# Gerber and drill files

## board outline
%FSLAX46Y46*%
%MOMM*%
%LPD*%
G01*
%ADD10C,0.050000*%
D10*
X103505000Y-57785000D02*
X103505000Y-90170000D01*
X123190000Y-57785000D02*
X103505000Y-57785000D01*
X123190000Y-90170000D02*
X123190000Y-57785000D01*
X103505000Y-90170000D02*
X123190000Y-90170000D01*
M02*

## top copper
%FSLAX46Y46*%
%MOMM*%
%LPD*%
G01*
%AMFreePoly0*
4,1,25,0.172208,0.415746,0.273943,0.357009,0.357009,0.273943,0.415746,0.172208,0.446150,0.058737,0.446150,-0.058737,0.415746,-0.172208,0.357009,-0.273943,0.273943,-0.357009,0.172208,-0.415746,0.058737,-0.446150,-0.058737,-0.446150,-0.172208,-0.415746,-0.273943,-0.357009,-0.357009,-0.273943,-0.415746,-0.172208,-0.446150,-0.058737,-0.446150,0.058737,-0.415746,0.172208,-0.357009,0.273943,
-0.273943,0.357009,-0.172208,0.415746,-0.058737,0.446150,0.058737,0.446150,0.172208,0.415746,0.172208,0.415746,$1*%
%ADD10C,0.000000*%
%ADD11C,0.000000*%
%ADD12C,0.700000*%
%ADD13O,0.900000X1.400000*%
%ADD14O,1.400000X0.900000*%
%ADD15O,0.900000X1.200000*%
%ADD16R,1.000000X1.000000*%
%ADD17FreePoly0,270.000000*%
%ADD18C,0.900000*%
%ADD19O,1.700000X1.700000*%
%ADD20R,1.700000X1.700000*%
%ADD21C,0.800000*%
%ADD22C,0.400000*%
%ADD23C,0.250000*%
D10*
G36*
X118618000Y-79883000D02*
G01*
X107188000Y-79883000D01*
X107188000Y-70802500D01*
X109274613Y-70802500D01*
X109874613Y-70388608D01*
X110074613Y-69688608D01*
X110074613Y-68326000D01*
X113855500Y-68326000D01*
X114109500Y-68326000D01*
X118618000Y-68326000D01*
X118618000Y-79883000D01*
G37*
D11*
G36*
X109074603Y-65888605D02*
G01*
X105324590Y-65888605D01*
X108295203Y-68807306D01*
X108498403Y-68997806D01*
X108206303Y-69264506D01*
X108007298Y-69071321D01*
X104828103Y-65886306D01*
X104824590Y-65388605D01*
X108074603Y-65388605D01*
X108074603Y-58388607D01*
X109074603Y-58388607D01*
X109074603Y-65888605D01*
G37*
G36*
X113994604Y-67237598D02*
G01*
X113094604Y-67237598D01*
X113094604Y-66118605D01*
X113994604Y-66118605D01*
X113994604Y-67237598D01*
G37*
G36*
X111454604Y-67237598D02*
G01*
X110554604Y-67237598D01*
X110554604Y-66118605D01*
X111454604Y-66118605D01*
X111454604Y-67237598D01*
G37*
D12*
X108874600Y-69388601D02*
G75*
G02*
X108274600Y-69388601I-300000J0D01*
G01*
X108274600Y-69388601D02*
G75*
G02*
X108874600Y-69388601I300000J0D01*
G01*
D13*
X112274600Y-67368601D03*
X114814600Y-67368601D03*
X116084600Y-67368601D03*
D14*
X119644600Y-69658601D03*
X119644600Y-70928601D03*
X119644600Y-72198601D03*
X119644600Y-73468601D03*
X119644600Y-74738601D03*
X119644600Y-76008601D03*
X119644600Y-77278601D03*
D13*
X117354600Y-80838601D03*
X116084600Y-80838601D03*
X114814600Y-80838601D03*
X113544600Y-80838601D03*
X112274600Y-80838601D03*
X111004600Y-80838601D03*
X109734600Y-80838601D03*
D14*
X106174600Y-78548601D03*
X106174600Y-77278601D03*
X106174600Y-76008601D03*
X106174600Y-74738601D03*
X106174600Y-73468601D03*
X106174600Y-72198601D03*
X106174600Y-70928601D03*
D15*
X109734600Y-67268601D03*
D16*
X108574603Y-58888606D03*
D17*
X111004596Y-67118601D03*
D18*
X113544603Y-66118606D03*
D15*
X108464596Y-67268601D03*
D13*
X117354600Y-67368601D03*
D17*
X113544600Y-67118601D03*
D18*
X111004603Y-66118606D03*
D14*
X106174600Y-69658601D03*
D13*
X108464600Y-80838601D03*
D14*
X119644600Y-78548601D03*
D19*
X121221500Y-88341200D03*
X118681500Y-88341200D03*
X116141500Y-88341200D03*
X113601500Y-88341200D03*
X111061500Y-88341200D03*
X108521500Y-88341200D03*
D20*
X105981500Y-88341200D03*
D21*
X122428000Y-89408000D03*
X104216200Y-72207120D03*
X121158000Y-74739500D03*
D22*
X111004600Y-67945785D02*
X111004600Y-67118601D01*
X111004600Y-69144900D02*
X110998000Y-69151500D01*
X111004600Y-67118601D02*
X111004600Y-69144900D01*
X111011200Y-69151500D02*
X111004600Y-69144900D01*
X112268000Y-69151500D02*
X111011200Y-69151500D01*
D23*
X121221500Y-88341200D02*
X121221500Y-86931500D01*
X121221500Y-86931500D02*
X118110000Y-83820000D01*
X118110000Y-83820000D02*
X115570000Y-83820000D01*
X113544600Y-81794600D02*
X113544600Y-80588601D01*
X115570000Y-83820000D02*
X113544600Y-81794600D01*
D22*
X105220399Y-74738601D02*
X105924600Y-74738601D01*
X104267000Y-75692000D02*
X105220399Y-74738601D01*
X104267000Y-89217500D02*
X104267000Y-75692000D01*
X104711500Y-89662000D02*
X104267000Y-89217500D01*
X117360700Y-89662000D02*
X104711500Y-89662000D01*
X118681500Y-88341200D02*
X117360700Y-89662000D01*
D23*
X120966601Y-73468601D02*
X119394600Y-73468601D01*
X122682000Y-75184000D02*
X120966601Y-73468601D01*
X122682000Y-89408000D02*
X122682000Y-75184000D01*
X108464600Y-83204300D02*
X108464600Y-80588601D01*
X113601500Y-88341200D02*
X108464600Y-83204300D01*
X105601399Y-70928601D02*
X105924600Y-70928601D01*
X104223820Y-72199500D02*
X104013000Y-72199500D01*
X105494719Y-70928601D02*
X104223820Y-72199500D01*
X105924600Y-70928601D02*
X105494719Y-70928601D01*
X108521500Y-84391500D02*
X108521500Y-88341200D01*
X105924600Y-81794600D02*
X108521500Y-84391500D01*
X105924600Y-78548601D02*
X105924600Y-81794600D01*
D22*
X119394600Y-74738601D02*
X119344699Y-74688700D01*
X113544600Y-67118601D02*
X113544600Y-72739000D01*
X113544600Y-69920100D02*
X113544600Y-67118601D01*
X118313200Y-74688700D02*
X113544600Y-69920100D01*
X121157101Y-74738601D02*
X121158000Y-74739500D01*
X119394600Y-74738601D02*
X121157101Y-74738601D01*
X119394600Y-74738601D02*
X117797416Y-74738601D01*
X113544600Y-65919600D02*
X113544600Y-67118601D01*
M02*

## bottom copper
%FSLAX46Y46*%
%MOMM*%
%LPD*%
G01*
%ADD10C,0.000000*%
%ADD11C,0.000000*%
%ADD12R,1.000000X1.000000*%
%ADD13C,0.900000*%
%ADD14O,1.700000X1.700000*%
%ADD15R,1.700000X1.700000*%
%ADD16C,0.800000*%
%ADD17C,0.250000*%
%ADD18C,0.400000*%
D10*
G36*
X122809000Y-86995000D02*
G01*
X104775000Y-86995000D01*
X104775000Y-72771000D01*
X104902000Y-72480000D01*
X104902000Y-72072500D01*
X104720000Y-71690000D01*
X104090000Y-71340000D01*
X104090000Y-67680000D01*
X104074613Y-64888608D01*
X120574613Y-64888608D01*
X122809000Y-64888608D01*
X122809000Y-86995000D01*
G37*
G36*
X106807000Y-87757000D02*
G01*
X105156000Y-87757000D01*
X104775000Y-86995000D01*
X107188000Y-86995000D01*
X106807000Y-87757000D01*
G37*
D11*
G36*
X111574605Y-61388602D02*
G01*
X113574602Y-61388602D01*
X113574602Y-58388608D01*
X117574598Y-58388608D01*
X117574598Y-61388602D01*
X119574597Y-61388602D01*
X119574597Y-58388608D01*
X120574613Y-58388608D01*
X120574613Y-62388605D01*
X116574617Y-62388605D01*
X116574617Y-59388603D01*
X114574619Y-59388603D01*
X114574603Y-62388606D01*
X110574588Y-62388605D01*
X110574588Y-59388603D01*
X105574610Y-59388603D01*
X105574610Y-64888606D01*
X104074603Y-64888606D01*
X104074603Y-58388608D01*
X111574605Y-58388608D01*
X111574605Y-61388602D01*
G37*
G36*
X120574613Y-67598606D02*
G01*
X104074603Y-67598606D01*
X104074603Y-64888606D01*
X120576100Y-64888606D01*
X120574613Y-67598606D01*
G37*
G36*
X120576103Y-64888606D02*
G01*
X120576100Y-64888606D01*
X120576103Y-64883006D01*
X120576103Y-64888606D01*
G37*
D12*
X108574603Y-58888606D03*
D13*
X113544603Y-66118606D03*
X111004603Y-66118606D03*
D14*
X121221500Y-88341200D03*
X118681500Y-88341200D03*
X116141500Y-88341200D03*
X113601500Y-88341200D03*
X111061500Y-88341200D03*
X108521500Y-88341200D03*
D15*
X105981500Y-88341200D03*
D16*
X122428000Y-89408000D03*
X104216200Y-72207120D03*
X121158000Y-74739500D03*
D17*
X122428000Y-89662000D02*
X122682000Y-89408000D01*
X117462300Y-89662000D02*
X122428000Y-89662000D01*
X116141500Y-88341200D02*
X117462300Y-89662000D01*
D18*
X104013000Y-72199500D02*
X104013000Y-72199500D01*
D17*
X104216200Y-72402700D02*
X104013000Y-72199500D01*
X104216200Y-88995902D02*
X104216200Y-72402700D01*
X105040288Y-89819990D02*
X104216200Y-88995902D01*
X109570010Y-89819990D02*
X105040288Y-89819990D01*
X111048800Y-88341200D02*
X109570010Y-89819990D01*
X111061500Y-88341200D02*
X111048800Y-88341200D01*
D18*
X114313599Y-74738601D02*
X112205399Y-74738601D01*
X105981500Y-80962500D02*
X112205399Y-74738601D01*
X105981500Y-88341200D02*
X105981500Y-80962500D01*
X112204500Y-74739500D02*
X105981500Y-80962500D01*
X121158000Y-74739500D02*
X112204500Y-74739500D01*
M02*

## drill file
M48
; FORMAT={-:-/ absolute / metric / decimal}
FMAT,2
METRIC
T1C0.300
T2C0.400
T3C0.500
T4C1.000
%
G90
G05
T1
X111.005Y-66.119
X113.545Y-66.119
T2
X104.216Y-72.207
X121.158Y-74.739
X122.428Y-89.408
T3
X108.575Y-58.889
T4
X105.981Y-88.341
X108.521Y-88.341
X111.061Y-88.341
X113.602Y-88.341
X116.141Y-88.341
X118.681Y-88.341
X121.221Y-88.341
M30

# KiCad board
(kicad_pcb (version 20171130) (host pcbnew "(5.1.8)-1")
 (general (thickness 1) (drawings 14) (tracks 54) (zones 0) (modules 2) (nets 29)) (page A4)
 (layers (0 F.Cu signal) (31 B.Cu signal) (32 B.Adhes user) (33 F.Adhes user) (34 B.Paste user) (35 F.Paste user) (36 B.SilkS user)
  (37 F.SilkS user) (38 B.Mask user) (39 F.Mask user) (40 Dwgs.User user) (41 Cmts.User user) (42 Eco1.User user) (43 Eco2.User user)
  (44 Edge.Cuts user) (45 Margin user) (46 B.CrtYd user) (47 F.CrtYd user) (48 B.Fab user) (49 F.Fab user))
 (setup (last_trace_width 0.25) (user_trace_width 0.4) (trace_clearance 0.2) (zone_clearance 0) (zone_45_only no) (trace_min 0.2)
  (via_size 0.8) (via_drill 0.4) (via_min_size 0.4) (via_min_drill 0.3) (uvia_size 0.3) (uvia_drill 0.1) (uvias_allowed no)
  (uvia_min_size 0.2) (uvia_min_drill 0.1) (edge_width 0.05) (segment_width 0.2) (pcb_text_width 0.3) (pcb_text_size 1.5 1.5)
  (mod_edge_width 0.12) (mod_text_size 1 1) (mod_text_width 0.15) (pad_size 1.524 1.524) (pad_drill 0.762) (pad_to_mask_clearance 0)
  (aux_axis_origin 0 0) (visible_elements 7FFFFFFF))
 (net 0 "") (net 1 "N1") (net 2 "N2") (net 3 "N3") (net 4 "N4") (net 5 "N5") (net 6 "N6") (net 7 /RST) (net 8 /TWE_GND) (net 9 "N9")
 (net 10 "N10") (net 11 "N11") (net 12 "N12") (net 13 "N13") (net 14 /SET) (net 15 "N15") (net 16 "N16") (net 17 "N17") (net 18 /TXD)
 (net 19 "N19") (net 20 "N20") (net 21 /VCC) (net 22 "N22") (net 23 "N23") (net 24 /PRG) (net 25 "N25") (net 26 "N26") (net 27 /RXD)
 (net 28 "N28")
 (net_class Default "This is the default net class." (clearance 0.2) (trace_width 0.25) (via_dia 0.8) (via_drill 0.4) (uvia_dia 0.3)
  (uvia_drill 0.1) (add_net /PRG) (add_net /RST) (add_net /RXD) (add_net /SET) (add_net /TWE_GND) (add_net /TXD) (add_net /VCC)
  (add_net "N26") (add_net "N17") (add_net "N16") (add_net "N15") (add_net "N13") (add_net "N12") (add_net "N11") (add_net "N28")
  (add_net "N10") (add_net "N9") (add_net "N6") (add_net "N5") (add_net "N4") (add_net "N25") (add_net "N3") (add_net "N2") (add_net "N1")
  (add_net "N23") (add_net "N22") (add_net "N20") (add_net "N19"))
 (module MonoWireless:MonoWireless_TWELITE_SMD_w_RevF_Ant (layer F.Cu) (at 112.9096 74.103601)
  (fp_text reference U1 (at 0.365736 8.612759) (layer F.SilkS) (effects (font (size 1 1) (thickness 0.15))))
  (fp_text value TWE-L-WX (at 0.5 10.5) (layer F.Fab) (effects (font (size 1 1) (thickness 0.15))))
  (fp_poly
   (pts (xy -1.334995 -12.714999) (xy 0.665002 -12.714999) (xy 0.665002 -15.714993) (xy 4.664998 -15.714993) (xy 4.664998 -12.714999)
    (xy 6.664997 -12.714999) (xy 6.664997 -15.714993) (xy 7.665013 -15.714993) (xy 7.665013 -11.714996) (xy 3.665017 -11.714996)
    (xy 3.665017 -14.714998) (xy 1.665019 -14.714998) (xy 1.665003 -11.714995) (xy -2.335012 -11.714996) (xy -2.335012 -14.714998)
    (xy -7.33499 -14.714998) (xy -7.33499 -9.214995) (xy -8.834997 -9.214995) (xy -8.834997 -15.714993) (xy -1.334995 -15.714993))
   (layer B.Cu) (width 0))
  (fp_poly
   (pts (xy 7.666503 -9.214995) (xy -8.834997 -9.214995) (xy -8.834997 -6.504995) (xy 7.665013 -6.504995) (xy 7.666503 -9.220595))
   (layer B.Cu) (width 0))
  (fp_poly
   (pts (xy -3.834997 -8.214996) (xy -7.58501 -8.214996) (xy -4.614397 -5.296295) (xy -4.411197 -5.105795) (xy -4.703297 -4.839095)
    (xy -4.902302 -5.03228) (xy -8.081497 -8.217295) (xy -8.08501 -8.714996) (xy -4.834997 -8.714996) (xy -4.834997 -15.714994)
    (xy -3.834997 -15.714994))
   (layer F.Cu) (width 0))
  (fp_poly (pts (xy 1.085004 -6.866003) (xy 0.185004 -6.866003) (xy 0.185004 -7.984996) (xy 1.085004 -7.984996)) (layer F.Cu) (width 0))
  (fp_poly (pts (xy -1.454996 -6.866003) (xy -2.354996 -6.866003) (xy -2.354996 -7.984996) (xy -1.454996 -7.984996)) (layer F.Cu) (width 0))
  (fp_circle (center -4.335 -4.715) (end -4.035 -4.715) (layer F.Cu) (width 0.7))
  (pad 29 smd oval (at -0.635 -6.735 90) (size 1.4 0.9) (layers F.Cu F.Paste F.Mask) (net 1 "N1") (zone_connect 0))
  (pad 27 smd oval (at 1.905 -6.735 90) (size 1.4 0.9) (layers F.Cu F.Paste F.Mask) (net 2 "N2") (zone_connect 0))
  (pad 26 smd oval (at 3.175 -6.735 90) (size 1.4 0.9) (layers F.Cu F.Paste F.Mask) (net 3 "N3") (zone_connect 0))
  (pad 24 smd oval (at 6.735 -4.445) (size 1.4 0.9) (layers F.Cu F.Paste F.Mask) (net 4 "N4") (zone_connect 0))
  (pad 23 smd oval (at 6.735 -3.175) (size 1.4 0.9) (layers F.Cu F.Paste F.Mask) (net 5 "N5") (zone_connect 0))
  (pad 22 smd oval (at 6.735 -1.905) (size 1.4 0.9) (layers F.Cu F.Paste F.Mask) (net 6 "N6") (zone_connect 0))
  (pad 21 smd oval (at 6.735 -0.635) (size 1.4 0.9) (layers F.Cu F.Paste F.Mask) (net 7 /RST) (zone_connect 0))
  (pad 20 smd oval (at 6.735 0.635) (size 1.4 0.9) (layers F.Cu F.Paste F.Mask) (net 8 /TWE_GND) (zone_connect 0))
  (pad 19 smd oval (at 6.735 1.905) (size 1.4 0.9) (layers F.Cu F.Paste F.Mask) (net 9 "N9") (zone_connect 0))
  (pad 18 smd oval (at 6.735 3.175) (size 1.4 0.9) (layers F.Cu F.Paste F.Mask) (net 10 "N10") (zone_connect 0))
  (pad 16 smd oval (at 4.445 6.735 270) (size 1.4 0.9) (layers F.Cu F.Paste F.Mask) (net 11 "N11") (zone_connect 0))
  (pad 15 smd oval (at 3.175 6.735 270) (size 1.4 0.9) (layers F.Cu F.Paste F.Mask) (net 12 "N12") (zone_connect 0))
  (pad 14 smd oval (at 1.905 6.735 270) (size 1.4 0.9) (layers F.Cu F.Paste F.Mask) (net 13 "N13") (zone_connect 0))
  (pad 13 smd oval (at 0.635 6.735 270) (size 1.4 0.9) (layers F.Cu F.Paste F.Mask) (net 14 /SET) (zone_connect 0))
  (pad 12 smd oval (at -0.635 6.735 270) (size 1.4 0.9) (layers F.Cu F.Paste F.Mask) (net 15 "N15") (zone_connect 0))
  (pad 11 smd oval (at -1.905 6.735 270) (size 1.4 0.9) (layers F.Cu F.Paste F.Mask) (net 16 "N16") (zone_connect 0))
  (pad 10 smd oval (at -3.175 6.735 270) (size 1.4 0.9) (layers F.Cu F.Paste F.Mask) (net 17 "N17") (zone_connect 0))
  (pad 8 smd oval (at -6.735 4.445) (size 1.4 0.9) (layers F.Cu F.Paste F.Mask) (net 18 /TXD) (zone_connect 0))
  (pad 7 smd oval (at -6.735 3.175) (size 1.4 0.9) (layers F.Cu F.Paste F.Mask) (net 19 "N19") (zone_connect 0))
  (pad 6 smd oval (at -6.735 1.905) (size 1.4 0.9) (layers F.Cu F.Paste F.Mask) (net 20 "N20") (zone_connect 0))
  (pad 5 smd oval (at -6.735 0.635) (size 1.4 0.9) (layers F.Cu F.Paste F.Mask) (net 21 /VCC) (zone_connect 0))
  (pad 4 smd oval (at -6.735 -0.635) (size 1.4 0.9) (layers F.Cu F.Paste F.Mask) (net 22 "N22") (zone_connect 0))
  (pad 3 smd oval (at -6.735 -1.905) (size 1.4 0.9) (layers F.Cu F.Paste F.Mask) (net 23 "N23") (zone_connect 0))
  (pad 2 smd oval (at -6.735 -3.175) (size 1.4 0.9) (layers F.Cu F.Paste F.Mask) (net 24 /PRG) (zone_connect 0))
  (pad 31 smd oval (at -3.175 -6.835 270) (size 1.2 0.9) (layers F.Cu F.Paste F.Mask) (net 8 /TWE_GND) (zone_connect 0))
  (pad "" thru_hole rect (at -4.334997 -15.214995 270) (size 1 1) (drill 0.5) (layers *.Cu *.Mask) (zone_connect 0))
  (pad "" smd custom (at -1.905004 -6.985 270) (size 0.9 0.9) (layers F.Cu F.Paste F.Mask) (zone_connect 0)
   (options (clearance outline) (anchor circle)) (primitives))
  (pad 28 thru_hole circle (at 0.635003 -7.984995 270) (size 0.9 0.9) (drill 0.3) (layers *.Cu) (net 8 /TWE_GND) (zone_connect 0))
  (pad 32 smd oval (at -4.445004 -6.835 270) (size 1.2 0.9) (layers F.Cu F.Paste F.Mask) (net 8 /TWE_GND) (zone_connect 0))
  (pad 25 smd oval (at 4.445 -6.735 90) (size 1.4 0.9) (layers F.Cu F.Paste F.Mask) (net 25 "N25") (zone_connect 0))
  (pad "" smd custom (at 0.635 -6.985 270) (size 0.9 0.9) (layers F.Cu F.Paste F.Mask) (zone_connect 0)
   (options (clearance outline) (anchor circle)) (primitives))
  (pad 30 thru_hole circle (at -1.904997 -7.984995 270) (size 0.9 0.9) (drill 0.3) (layers *.Cu) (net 8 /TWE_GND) (zone_connect 0))
  (pad 1 smd oval (at -6.735 -4.445) (size 1.4 0.9) (layers F.Cu F.Paste F.Mask) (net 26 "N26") (zone_connect 0))
  (pad 9 smd oval (at -4.445 6.735 270) (size 1.4 0.9) (layers F.Cu F.Paste F.Mask) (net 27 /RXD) (zone_connect 0))
  (pad 17 smd oval (at 6.735 4.445) (size 1.4 0.9) (layers F.Cu F.Paste F.Mask) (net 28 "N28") (zone_connect 0)))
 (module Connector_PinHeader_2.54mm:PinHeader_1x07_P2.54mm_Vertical (layer F.Cu) (at 105.9815 88.3412 90)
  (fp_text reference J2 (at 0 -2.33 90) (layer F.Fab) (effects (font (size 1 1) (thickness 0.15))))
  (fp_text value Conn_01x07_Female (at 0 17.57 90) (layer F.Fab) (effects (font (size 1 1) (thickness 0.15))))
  (pad 7 thru_hole oval (at 0 15.24 90) (size 1.7 1.7) (drill 1) (layers *.Cu *.Mask) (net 14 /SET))
  (pad 6 thru_hole oval (at 0 12.7 90) (size 1.7 1.7) (drill 1) (layers *.Cu *.Mask) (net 21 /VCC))
  (pad 5 thru_hole oval (at 0 10.16 90) (size 1.7 1.7) (drill 1) (layers *.Cu *.Mask) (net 7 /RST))
  (pad 4 thru_hole oval (at 0 7.62 90) (size 1.7 1.7) (drill 1) (layers *.Cu *.Mask) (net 27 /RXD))
  (pad 3 thru_hole oval (at 0 5.08 90) (size 1.7 1.7) (drill 1) (layers *.Cu *.Mask) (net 24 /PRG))
  (pad 2 thru_hole oval (at 0 2.54 90) (size 1.7 1.7) (drill 1) (layers *.Cu *.Mask) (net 18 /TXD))
  (pad 1 thru_hole rect (at 0 0 90) (size 1.7 1.7) (drill 1) (layers *.Cu *.Mask) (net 8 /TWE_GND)))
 (gr_poly
  (pts (xy 122.809 86.995) (xy 104.775 86.995) (xy 104.775 72.771) (xy 104.902 72.48) (xy 104.902 72.0725) (xy 104.72 71.69)
   (xy 104.09 71.34) (xy 104.09 67.68) (xy 104.074613 64.888608) (xy 120.574613 64.888608) (xy 122.809 64.888608))
  (layer B.Cu) (width 0))
 (gr_poly (pts (xy 106.807 87.757) (xy 105.156 87.757) (xy 104.775 86.995) (xy 107.188 86.995)) (layer B.Cu) (width 0))
 (gr_poly
  (pts (xy 113.8555 68.326) (xy 114.1095 68.326) (xy 118.618 68.326) (xy 118.618 79.883) (xy 107.188 79.883) (xy 107.188 70.8025)
   (xy 109.274613 70.8025) (xy 109.874613 70.388608) (xy 110.074613 69.688608) (xy 110.074613 68.326))
  (layer F.Cu) (width 0))
 (gr_line (start 103.505 57.785) (end 103.505 90.17) (layer Edge.Cuts) (width 0.05))
 (gr_line (start 123.19 57.785) (end 103.505 57.785) (layer Edge.Cuts) (width 0.05))
 (gr_line (start 123.19 90.17) (end 123.19 57.785) (layer Edge.Cuts) (width 0.05))
 (gr_line (start 103.505 90.17) (end 123.19 90.17) (layer Edge.Cuts) (width 0.05))
 (segment (start 111.0046 67.945785) (end 111.0046 67.118601) (width 0.4) (layer F.Cu) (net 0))
 (segment (start 111.0046 69.1449) (end 110.998 69.1515) (width 0.4) (layer F.Cu) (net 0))
 (segment (start 111.0046 67.118601) (end 111.0046 69.1449) (width 0.4) (layer F.Cu) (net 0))
 (segment (start 111.0112 69.1515) (end 111.0046 69.1449) (width 0.4) (layer F.Cu) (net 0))
 (segment (start 112.268 69.1515) (end 111.0112 69.1515) (width 0.4) (layer F.Cu) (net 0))
 (segment (start 121.2215 88.3412) (end 121.2215 86.9315) (width 0.25) (layer F.Cu) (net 14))
 (segment (start 121.2215 86.9315) (end 118.11 83.82) (width 0.25) (layer F.Cu) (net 14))
 (segment (start 118.11 83.82) (end 115.57 83.82) (width 0.25) (layer F.Cu) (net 14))
 (segment (start 113.5446 81.7946) (end 113.5446 80.588601) (width 0.25) (layer F.Cu) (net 14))
 (segment (start 115.57 83.82) (end 113.5446 81.7946) (width 0.25) (layer F.Cu) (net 14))
 (segment (start 105.220399 74.738601) (end 105.9246 74.738601) (width 0.4) (layer F.Cu) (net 21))
 (segment (start 104.267 75.692) (end 105.220399 74.738601) (width 0.4) (layer F.Cu) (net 21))
 (segment (start 104.267 89.2175) (end 104.267 75.692) (width 0.4) (layer F.Cu) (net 21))
 (segment (start 104.7115 89.662) (end 104.267 89.2175) (width 0.4) (layer F.Cu) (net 21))
 (segment (start 117.3607 89.662) (end 104.7115 89.662) (width 0.4) (layer F.Cu) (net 21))
 (segment (start 118.6815 88.3412) (end 117.3607 89.662) (width 0.4) (layer F.Cu) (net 21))
 (via (at 122.428 89.408) (size 0.8) (drill 0.4) (layers F.Cu B.Cu) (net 7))
 (segment (start 120.966601 73.468601) (end 119.3946 73.468601) (width 0.25) (layer F.Cu) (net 7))
 (segment (start 122.682 75.184) (end 120.966601 73.468601) (width 0.25) (layer F.Cu) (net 7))
 (segment (start 122.682 89.408) (end 122.682 75.184) (width 0.25) (layer F.Cu) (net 7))
 (segment (start 122.428 89.662) (end 122.682 89.408) (width 0.25) (layer B.Cu) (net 7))
 (segment (start 117.4623 89.662) (end 122.428 89.662) (width 0.25) (layer B.Cu) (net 7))
 (segment (start 116.1415 88.3412) (end 117.4623 89.662) (width 0.25) (layer B.Cu) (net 7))
 (segment (start 108.4646 83.2043) (end 108.4646 80.588601) (width 0.25) (layer F.Cu) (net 27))
 (segment (start 113.6015 88.3412) (end 108.4646 83.2043) (width 0.25) (layer F.Cu) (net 27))
 (segment (start 105.601399 70.928601) (end 105.9246 70.928601) (width 0.25) (layer F.Cu) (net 24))
 (segment (start 104.013 72.1995) (end 104.013 72.1995) (width 0.4) (layer B.Cu) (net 24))
 (via (at 104.2162 72.20712) (size 0.8) (drill 0.4) (layers F.Cu B.Cu) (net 24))
 (segment (start 104.22382 72.1995) (end 104.013 72.1995) (width 0.25) (layer F.Cu) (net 24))
 (segment (start 105.494719 70.928601) (end 104.22382 72.1995) (width 0.25) (layer F.Cu) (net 24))
 (segment (start 105.9246 70.928601) (end 105.494719 70.928601) (width 0.25) (layer F.Cu) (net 24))
 (segment (start 104.2162 72.4027) (end 104.013 72.1995) (width 0.25) (layer B.Cu) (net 24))
 (segment (start 104.2162 88.995902) (end 104.2162 72.4027) (width 0.25) (layer B.Cu) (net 24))
 (segment (start 105.040288 89.81999) (end 104.2162 88.995902) (width 0.25) (layer B.Cu) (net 24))
 (segment (start 109.57001 89.81999) (end 105.040288 89.81999) (width 0.25) (layer B.Cu) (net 24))
 (segment (start 111.0488 88.3412) (end 109.57001 89.81999) (width 0.25) (layer B.Cu) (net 24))
 (segment (start 111.0615 88.3412) (end 111.0488 88.3412) (width 0.25) (layer B.Cu) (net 24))
 (segment (start 108.5215 84.3915) (end 108.5215 88.3412) (width 0.25) (layer F.Cu) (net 18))
 (segment (start 105.9246 81.7946) (end 108.5215 84.3915) (width 0.25) (layer F.Cu) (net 18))
 (segment (start 105.9246 78.548601) (end 105.9246 81.7946) (width 0.25) (layer F.Cu) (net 18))
 (segment (start 114.313599 74.738601) (end 112.205399 74.738601) (width 0.4) (layer B.Cu) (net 8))
 (via (at 121.158 74.7395) (size 0.8) (drill 0.4) (layers F.Cu B.Cu) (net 8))
 (segment (start 119.3946 74.738601) (end 119.344699 74.6887) (width 0.4) (layer F.Cu) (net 8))
 (segment (start 113.5446 67.118601) (end 113.5446 72.739) (width 0.4) (layer F.Cu) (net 8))
 (segment (start 113.5446 69.9201) (end 113.5446 67.118601) (width 0.4) (layer F.Cu) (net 8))
 (segment (start 118.3132 74.6887) (end 113.5446 69.9201) (width 0.4) (layer F.Cu) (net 8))
 (segment (start 105.9815 80.9625) (end 112.205399 74.738601) (width 0.4) (layer B.Cu) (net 8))
 (segment (start 105.9815 88.3412) (end 105.9815 80.9625) (width 0.4) (layer B.Cu) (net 8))
 (segment (start 121.157101 74.738601) (end 121.158 74.7395) (width 0.4) (layer F.Cu) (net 8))
 (segment (start 119.3946 74.738601) (end 121.157101 74.738601) (width 0.4) (layer F.Cu) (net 8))
 (segment (start 112.2045 74.7395) (end 105.9815 80.9625) (width 0.4) (layer B.Cu) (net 8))
 (segment (start 121.158 74.7395) (end 112.2045 74.7395) (width 0.4) (layer B.Cu) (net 8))
 (segment (start 119.3946 74.738601) (end 117.797416 74.738601) (width 0.4) (layer F.Cu) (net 8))
 (segment (start 113.5446 65.9196) (end 113.5446 67.118601) (width 0.4) (layer F.Cu) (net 8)))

